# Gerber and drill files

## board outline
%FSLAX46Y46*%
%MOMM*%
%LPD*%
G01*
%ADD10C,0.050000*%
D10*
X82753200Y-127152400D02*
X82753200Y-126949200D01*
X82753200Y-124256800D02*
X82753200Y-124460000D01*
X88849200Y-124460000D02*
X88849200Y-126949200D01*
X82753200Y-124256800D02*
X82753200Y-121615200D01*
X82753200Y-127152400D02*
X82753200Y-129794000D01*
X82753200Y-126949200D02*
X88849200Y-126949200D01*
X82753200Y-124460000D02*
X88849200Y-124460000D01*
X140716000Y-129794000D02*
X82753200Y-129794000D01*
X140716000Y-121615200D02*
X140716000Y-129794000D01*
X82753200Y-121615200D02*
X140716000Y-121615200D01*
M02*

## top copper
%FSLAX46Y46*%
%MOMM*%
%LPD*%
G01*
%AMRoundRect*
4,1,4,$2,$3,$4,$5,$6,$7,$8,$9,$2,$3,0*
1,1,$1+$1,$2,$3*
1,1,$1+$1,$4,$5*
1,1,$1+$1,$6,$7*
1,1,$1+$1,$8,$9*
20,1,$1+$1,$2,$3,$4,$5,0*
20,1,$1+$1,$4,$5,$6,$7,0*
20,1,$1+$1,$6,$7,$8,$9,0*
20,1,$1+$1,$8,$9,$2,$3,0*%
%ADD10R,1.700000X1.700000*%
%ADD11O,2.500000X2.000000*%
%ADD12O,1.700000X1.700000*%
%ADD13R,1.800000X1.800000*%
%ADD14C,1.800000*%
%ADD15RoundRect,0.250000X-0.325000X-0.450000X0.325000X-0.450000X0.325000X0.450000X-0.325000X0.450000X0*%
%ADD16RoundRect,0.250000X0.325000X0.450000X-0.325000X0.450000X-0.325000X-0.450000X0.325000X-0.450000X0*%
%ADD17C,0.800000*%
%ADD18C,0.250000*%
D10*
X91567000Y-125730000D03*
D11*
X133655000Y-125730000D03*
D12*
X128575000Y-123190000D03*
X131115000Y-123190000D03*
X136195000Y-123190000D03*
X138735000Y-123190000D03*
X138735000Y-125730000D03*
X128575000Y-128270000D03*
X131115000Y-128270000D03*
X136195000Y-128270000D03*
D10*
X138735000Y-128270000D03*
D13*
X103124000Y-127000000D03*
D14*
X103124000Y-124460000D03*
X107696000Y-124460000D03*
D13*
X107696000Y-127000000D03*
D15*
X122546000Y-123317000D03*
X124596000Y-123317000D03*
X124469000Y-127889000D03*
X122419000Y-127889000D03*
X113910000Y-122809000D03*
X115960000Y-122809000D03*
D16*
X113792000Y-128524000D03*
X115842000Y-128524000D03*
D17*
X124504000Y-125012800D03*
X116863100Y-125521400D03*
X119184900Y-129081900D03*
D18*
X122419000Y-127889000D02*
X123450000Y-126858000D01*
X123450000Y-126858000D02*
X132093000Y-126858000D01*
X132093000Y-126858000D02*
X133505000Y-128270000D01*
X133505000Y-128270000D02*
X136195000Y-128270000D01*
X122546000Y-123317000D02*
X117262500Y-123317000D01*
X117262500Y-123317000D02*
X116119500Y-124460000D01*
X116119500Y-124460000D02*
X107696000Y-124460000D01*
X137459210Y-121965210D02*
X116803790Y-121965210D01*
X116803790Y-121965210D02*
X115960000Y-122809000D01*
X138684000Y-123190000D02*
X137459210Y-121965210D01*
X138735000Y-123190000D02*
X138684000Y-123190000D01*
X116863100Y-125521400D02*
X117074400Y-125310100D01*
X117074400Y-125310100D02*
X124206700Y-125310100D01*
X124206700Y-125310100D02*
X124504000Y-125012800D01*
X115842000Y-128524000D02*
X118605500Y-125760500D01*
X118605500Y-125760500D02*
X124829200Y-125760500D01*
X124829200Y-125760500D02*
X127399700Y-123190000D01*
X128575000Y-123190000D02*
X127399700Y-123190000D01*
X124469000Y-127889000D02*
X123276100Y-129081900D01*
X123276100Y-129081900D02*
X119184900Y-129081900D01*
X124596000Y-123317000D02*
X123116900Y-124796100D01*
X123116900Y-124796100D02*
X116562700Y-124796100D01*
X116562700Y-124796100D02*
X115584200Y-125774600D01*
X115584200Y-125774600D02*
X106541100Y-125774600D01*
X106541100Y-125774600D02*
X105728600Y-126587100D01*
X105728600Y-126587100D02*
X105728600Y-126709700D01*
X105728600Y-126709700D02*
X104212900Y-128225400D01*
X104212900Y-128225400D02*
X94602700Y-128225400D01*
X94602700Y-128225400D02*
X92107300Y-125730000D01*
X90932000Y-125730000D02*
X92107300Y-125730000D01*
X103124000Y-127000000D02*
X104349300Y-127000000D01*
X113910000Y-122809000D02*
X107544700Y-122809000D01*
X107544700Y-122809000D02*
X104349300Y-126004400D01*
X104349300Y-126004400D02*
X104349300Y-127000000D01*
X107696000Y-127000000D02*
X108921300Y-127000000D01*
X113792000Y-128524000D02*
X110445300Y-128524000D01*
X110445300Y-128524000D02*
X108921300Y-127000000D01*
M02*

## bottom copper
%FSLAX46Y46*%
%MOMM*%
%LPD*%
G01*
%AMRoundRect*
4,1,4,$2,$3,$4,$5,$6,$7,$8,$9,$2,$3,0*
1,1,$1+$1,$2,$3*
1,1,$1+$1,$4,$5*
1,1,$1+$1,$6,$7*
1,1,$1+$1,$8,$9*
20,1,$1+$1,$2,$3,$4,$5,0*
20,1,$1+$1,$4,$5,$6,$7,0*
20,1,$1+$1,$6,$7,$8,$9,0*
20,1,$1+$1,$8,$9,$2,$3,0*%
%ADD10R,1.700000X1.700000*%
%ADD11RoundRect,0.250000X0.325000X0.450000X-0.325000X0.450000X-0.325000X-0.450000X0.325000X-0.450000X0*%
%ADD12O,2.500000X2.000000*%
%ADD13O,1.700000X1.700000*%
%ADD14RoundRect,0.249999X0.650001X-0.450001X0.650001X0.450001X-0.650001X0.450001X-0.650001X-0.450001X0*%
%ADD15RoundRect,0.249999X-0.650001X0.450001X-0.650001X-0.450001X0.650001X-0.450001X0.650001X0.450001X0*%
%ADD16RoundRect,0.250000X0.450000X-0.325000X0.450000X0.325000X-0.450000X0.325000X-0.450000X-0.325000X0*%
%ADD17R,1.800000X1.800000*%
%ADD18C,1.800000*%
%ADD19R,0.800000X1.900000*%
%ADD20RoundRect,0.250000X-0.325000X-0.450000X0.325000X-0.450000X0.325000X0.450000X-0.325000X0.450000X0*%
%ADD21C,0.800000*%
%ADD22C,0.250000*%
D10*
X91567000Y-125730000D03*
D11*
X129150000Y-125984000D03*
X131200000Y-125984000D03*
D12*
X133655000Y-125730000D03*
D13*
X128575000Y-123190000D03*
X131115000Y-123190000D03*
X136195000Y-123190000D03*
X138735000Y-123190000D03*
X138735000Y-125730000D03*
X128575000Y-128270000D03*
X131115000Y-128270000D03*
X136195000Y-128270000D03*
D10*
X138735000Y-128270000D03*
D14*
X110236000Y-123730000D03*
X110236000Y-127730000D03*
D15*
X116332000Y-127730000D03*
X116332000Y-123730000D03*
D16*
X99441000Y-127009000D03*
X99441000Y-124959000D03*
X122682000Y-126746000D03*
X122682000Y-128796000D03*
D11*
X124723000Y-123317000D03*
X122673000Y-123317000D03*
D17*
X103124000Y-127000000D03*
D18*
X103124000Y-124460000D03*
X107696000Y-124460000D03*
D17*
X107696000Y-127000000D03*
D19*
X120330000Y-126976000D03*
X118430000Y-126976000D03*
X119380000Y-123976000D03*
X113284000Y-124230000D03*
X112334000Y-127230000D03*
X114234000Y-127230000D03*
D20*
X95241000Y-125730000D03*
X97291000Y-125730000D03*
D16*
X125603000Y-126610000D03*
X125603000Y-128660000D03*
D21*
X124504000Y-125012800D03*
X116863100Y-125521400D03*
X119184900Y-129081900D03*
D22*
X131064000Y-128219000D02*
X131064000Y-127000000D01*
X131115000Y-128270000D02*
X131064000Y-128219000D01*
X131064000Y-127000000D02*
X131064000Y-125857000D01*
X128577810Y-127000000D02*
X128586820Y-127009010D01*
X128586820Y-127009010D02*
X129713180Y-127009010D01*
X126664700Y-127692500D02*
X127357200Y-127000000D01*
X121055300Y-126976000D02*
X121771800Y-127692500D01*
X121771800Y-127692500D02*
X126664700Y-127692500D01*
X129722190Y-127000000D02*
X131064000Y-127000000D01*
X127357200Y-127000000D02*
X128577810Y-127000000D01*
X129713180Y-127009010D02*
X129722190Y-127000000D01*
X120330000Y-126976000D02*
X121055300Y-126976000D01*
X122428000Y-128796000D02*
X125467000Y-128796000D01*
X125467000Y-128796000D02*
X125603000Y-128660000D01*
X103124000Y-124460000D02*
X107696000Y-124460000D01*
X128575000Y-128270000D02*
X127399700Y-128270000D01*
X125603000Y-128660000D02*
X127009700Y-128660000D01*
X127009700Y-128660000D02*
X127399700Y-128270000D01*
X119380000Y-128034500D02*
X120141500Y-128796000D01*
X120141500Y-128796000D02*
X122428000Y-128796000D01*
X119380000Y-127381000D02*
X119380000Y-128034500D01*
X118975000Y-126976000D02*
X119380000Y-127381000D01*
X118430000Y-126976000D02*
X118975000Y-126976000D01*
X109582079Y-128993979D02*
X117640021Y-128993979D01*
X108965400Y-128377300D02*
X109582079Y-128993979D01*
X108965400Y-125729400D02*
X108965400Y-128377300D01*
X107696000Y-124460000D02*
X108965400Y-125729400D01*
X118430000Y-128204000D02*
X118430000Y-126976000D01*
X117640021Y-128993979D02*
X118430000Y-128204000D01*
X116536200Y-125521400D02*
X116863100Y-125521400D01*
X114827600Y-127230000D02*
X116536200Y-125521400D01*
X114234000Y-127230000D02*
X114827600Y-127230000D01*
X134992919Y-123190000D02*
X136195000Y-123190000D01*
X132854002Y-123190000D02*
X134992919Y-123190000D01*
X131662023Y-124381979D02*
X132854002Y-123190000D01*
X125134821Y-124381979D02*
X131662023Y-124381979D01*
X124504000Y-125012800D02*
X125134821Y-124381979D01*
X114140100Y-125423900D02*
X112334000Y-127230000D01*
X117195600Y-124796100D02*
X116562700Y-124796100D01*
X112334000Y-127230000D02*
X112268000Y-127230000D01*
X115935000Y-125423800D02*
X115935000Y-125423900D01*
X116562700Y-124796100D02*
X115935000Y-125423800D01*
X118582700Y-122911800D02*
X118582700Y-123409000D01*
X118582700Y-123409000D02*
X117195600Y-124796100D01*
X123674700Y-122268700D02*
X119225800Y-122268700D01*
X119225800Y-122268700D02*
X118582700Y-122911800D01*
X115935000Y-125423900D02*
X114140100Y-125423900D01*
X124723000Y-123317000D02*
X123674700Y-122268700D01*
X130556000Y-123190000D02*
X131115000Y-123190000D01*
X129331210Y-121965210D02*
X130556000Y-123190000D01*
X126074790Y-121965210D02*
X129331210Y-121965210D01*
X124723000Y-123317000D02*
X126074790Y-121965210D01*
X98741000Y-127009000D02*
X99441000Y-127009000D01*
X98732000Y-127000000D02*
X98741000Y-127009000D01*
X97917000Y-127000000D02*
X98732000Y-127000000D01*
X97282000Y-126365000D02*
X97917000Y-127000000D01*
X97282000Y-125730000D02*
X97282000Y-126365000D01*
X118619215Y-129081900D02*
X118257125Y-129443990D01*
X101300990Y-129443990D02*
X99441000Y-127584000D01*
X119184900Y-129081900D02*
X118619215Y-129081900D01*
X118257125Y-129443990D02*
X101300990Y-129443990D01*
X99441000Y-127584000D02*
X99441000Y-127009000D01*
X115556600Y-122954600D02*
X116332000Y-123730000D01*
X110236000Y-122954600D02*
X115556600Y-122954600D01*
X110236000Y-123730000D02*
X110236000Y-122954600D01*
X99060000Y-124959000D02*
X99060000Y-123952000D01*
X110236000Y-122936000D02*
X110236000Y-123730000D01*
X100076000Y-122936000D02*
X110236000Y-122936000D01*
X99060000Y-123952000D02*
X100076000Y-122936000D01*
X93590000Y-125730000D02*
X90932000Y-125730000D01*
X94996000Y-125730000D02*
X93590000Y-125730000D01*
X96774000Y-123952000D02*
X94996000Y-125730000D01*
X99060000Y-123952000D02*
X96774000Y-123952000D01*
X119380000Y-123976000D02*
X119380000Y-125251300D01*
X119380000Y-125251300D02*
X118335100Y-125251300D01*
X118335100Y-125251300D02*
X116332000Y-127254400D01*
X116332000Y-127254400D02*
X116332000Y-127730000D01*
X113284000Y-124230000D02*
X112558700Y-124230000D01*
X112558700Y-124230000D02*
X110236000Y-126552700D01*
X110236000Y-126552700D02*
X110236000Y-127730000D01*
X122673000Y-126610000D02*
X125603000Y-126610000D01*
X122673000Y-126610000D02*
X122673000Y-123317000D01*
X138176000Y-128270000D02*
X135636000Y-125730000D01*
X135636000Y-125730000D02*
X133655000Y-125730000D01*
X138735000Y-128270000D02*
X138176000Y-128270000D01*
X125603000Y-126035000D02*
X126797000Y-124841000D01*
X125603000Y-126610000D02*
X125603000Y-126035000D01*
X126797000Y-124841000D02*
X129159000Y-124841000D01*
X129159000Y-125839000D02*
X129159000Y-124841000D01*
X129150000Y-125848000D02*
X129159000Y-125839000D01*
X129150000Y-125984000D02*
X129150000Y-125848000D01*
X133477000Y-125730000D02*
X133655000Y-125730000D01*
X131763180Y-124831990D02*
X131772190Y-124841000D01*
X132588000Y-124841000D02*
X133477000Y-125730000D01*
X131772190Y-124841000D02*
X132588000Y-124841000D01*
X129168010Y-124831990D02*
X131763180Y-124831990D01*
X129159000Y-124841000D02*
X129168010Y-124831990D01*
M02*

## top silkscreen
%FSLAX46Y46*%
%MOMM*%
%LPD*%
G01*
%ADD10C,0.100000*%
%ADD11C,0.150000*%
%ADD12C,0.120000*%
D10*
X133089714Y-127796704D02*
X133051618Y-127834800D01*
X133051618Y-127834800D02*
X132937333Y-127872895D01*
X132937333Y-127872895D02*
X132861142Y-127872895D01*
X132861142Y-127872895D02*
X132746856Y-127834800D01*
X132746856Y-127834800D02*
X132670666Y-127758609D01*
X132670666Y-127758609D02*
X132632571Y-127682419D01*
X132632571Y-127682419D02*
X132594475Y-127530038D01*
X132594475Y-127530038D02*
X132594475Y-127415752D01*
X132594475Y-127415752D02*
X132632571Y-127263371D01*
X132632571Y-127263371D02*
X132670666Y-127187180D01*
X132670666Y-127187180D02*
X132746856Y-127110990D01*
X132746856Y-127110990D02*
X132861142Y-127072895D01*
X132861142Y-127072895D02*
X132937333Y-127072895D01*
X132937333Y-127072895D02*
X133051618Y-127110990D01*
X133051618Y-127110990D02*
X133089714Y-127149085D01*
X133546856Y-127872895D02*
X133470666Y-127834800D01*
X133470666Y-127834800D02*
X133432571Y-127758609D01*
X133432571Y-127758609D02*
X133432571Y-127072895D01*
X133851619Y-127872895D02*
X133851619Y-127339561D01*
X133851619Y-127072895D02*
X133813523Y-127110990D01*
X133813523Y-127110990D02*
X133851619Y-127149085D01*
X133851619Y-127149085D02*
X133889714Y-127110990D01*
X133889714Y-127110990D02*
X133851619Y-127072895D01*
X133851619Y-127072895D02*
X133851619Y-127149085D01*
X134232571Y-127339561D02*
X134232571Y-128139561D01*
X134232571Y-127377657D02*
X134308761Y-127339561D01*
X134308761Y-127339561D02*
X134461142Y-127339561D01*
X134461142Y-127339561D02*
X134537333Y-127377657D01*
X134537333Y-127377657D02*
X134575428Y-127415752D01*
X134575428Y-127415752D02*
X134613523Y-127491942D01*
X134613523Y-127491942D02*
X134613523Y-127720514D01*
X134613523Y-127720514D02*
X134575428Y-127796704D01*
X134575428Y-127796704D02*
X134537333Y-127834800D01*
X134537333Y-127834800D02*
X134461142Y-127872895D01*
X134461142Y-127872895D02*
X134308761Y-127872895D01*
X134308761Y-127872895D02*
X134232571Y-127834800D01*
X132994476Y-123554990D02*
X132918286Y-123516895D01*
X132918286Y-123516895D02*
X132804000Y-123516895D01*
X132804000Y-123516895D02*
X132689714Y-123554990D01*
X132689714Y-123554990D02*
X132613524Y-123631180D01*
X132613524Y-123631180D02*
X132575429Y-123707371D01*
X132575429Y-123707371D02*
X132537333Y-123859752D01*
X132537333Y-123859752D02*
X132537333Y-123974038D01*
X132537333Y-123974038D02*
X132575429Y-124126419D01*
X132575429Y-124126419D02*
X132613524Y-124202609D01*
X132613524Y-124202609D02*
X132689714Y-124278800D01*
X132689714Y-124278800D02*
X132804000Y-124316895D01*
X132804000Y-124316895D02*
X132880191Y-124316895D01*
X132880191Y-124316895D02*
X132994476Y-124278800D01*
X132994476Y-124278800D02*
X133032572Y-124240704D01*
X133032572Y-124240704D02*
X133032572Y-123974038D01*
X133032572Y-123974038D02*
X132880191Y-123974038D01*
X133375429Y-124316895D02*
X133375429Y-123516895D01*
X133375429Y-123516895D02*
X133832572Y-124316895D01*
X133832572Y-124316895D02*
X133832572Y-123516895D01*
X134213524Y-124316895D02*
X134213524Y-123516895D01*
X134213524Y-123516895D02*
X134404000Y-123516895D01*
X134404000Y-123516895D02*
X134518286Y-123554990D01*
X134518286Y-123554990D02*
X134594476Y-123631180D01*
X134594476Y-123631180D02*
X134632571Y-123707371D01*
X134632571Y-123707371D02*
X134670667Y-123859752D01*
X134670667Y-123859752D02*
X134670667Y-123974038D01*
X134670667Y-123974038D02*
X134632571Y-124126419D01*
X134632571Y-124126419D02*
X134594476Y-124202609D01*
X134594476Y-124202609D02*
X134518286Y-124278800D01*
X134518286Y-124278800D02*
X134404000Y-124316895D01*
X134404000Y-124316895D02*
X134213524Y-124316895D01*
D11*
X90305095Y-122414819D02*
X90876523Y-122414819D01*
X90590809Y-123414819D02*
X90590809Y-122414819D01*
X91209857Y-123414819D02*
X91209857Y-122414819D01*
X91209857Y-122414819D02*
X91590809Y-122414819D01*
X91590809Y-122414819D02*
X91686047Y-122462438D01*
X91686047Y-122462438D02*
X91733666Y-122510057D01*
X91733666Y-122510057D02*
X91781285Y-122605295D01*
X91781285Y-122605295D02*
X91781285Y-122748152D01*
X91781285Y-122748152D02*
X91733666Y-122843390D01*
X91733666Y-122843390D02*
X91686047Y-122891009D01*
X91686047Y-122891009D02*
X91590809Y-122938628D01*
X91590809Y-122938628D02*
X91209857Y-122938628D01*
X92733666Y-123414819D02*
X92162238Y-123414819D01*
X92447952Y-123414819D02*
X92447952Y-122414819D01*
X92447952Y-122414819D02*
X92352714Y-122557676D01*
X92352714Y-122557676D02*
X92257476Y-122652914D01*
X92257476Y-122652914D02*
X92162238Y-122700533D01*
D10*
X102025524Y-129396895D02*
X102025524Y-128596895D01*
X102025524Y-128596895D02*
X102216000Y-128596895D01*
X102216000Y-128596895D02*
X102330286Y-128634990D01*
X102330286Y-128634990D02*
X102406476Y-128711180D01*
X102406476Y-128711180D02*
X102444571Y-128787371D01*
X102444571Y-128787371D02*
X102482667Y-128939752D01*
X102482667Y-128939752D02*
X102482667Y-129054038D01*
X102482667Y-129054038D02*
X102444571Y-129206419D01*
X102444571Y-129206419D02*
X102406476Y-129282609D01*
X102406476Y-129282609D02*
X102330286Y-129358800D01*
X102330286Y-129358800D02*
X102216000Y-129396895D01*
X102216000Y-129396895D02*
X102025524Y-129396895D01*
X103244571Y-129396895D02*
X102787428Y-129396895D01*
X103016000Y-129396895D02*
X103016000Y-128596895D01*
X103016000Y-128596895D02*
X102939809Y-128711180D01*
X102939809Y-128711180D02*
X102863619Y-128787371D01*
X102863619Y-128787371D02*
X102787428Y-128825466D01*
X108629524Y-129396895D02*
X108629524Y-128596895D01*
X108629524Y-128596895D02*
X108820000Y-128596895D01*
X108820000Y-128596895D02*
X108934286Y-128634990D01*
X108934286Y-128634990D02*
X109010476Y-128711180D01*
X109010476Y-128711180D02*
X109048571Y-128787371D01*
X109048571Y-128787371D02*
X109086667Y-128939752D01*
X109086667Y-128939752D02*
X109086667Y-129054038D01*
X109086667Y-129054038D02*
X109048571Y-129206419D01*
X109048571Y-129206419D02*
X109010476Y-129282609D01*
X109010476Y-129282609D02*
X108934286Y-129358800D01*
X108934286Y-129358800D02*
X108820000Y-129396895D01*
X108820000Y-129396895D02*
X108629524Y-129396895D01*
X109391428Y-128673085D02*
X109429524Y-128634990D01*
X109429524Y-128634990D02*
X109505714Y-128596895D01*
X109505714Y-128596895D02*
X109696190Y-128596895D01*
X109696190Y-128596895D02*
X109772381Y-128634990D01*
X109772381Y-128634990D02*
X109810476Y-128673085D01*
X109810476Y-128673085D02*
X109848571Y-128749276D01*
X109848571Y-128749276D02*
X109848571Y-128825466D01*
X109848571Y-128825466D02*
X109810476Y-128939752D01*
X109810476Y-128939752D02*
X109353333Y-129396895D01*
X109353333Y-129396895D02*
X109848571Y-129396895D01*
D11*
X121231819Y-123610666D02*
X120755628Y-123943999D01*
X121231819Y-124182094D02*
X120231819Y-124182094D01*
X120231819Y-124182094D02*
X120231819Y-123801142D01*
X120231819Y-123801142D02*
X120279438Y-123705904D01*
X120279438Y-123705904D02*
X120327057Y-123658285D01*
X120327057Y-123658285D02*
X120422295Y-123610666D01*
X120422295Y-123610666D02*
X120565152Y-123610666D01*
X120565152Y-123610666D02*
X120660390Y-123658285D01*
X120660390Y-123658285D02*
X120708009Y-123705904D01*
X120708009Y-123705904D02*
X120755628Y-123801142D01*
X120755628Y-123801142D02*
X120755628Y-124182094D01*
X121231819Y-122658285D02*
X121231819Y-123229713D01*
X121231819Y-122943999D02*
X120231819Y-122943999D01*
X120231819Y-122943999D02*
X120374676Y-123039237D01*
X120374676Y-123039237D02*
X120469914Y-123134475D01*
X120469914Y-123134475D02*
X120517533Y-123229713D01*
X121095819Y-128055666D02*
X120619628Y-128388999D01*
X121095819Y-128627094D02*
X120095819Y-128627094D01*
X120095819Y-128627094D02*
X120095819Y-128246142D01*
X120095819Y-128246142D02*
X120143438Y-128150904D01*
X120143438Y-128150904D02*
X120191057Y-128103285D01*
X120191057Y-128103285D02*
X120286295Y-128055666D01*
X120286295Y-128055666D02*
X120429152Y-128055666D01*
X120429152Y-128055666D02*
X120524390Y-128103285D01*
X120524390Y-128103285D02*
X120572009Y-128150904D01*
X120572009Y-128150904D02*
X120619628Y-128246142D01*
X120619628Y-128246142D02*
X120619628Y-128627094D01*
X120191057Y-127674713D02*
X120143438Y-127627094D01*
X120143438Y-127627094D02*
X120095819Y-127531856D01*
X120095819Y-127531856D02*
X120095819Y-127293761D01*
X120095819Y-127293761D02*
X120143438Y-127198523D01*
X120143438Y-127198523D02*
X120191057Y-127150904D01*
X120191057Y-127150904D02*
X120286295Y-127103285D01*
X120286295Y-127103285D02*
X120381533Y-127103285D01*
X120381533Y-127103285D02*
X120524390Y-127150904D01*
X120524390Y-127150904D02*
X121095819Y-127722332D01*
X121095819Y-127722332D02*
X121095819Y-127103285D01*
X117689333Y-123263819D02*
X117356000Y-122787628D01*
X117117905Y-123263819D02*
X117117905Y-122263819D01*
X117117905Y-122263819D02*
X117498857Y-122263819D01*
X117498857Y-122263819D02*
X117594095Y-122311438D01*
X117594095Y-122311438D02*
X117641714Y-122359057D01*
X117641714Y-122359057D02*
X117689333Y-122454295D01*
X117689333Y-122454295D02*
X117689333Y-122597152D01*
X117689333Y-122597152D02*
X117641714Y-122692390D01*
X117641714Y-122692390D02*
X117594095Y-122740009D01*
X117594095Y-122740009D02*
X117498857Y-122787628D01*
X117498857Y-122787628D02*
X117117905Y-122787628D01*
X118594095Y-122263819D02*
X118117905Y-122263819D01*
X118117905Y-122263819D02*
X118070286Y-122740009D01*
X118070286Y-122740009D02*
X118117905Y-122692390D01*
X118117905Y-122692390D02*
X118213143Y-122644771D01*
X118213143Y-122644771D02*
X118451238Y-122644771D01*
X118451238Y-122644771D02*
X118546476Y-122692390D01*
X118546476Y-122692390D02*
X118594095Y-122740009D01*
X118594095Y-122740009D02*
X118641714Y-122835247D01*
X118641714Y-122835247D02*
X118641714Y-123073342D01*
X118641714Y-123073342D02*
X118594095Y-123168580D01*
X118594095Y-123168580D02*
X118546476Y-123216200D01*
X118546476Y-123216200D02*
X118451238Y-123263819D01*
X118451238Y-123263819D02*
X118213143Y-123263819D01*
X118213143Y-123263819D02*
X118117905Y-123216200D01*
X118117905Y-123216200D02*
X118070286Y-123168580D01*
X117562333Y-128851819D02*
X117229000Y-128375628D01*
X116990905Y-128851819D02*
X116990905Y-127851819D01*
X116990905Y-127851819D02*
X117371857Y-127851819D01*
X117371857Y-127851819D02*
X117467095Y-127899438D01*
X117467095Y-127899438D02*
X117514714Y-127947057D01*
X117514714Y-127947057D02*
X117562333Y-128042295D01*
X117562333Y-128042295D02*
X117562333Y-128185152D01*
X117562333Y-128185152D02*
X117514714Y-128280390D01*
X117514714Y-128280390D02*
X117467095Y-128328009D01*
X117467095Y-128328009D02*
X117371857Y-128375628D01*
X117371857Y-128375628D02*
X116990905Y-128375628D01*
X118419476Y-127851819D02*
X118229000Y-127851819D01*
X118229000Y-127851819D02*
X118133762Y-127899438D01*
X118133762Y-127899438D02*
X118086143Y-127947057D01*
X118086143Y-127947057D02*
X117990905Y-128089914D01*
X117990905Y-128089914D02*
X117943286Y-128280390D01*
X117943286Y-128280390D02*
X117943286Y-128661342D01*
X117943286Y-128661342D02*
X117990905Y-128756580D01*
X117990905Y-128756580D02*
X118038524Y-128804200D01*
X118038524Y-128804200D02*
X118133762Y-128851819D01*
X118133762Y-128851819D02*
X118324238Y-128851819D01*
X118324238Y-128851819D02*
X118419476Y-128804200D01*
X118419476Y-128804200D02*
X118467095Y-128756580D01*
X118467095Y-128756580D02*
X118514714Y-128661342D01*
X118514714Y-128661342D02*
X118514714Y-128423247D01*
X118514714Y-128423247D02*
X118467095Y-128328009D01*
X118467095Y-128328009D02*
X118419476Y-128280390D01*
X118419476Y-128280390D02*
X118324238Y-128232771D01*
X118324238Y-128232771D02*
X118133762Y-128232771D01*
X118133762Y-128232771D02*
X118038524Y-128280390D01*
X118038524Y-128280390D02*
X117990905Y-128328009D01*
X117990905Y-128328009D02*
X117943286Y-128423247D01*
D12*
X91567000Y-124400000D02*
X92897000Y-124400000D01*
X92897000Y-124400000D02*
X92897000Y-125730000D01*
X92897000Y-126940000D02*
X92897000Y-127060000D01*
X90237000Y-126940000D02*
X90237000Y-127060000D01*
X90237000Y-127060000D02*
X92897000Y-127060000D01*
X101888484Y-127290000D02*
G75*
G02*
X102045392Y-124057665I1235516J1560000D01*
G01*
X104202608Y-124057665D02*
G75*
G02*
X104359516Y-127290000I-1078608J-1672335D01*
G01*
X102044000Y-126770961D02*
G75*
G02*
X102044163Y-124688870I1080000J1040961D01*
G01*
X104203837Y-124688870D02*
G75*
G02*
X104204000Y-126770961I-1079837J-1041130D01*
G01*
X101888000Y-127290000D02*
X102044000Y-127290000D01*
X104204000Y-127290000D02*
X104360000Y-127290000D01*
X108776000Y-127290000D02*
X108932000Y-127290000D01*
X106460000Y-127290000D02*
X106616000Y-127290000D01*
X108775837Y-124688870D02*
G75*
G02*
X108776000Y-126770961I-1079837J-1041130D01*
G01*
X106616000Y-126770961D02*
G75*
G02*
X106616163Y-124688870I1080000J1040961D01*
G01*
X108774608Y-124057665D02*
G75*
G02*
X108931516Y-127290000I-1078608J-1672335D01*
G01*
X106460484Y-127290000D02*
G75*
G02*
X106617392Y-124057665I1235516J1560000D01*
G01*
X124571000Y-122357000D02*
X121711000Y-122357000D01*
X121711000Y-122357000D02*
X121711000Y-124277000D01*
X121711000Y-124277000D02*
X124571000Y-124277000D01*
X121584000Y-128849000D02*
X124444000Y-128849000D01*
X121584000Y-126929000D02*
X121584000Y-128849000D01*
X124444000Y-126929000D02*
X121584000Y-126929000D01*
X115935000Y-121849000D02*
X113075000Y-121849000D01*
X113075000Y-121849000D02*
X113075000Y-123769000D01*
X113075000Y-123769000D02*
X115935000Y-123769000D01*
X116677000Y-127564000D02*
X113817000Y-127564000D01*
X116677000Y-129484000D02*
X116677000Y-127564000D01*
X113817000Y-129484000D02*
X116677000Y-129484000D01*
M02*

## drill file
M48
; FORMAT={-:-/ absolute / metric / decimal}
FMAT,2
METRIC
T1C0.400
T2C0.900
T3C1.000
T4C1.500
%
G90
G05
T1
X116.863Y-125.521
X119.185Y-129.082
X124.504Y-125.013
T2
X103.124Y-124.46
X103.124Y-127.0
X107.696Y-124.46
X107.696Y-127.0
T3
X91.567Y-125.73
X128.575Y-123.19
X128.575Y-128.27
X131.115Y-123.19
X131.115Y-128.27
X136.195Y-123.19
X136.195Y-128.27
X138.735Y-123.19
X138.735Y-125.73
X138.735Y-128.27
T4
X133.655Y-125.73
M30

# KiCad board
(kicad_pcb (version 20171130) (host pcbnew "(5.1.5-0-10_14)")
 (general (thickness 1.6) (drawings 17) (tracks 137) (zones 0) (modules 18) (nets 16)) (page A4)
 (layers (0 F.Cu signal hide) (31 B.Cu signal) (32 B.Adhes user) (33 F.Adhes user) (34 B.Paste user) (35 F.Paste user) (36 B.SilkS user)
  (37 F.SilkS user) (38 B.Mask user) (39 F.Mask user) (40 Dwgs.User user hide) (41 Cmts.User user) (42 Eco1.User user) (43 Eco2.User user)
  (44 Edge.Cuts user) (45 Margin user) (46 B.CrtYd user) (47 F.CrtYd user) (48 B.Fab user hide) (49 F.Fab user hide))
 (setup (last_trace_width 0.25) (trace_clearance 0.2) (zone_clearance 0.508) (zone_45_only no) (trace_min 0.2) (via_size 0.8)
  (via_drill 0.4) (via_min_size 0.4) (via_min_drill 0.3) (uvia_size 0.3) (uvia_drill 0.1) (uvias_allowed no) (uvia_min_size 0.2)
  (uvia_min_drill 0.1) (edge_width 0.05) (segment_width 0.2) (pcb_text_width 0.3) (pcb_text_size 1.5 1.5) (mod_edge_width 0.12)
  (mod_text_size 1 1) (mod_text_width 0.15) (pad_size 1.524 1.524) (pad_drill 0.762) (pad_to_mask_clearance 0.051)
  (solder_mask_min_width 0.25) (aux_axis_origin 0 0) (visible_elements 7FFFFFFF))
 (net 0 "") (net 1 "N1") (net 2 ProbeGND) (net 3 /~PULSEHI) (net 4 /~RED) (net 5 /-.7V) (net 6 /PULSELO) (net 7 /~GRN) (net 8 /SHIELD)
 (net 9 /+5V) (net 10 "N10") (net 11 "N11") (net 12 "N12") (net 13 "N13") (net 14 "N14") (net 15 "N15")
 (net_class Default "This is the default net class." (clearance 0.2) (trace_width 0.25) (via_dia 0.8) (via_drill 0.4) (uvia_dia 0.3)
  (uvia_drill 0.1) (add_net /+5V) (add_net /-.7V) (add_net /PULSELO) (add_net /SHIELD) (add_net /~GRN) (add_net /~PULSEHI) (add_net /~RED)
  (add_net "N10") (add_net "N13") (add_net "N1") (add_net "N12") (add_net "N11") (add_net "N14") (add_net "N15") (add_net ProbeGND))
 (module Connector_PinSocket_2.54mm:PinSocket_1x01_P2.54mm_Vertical (layer F.Cu) (at 91.567 125.73)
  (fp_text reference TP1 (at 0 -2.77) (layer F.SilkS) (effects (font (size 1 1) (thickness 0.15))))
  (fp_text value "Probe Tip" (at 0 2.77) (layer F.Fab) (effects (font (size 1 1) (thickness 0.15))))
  (fp_line (start 0 -1.33) (end 1.33 -1.33) (layer F.SilkS) (width 0.12))
  (fp_line (start 1.33 -1.33) (end 1.33 0) (layer F.SilkS) (width 0.12))
  (fp_line (start 1.33 1.21) (end 1.33 1.33) (layer F.SilkS) (width 0.12))
  (fp_line (start -1.33 1.21) (end -1.33 1.33) (layer F.SilkS) (width 0.12))
  (fp_line (start -1.33 1.33) (end 1.33 1.33) (layer F.SilkS) (width 0.12))
  (pad 1 thru_hole rect (at 0 0) (size 1.7 1.7) (drill 1) (layers *.Cu *.Mask) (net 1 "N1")))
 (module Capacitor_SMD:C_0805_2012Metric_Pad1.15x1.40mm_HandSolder (layer B.Cu) (at 130.175 125.984 180)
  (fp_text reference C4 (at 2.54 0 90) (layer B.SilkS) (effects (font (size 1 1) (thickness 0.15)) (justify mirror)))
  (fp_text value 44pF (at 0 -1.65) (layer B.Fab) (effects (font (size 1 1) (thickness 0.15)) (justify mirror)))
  (pad 2 smd roundrect (at 1.025 0 180) (size 1.15 1.4) (layers B.Cu B.Paste B.Mask) (roundrect_rratio 0.217391) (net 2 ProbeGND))
  (pad 1 smd roundrect (at -1.025 0 180) (size 1.15 1.4) (layers B.Cu B.Paste B.Mask) (roundrect_rratio 0.217391) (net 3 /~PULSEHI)))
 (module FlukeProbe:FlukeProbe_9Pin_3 (layer B.Cu) (at 138.735 128.27 90)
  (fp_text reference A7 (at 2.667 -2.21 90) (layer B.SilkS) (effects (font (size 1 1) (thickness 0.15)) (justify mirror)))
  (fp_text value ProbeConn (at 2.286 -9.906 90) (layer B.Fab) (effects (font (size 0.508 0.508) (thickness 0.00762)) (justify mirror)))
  (pad 10 thru_hole oval (at 2.54 -5.08 90) (size 2 2.5) (drill 1.5) (layers *.Cu *.Mask) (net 2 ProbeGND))
  (pad 9 thru_hole oval (at 5.08 -10.16 90) (size 1.7 1.7) (drill 1) (layers *.Cu *.Mask) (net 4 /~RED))
  (pad 8 thru_hole oval (at 5.08 -7.62 90) (size 1.7 1.7) (drill 1) (layers *.Cu *.Mask) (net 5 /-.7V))
  (pad 7 thru_hole oval (at 5.08 -2.54 90) (size 1.7 1.7) (drill 1) (layers *.Cu *.Mask) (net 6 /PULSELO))
  (pad 6 thru_hole oval (at 5.08 0 90) (size 1.7 1.7) (drill 1) (layers *.Cu *.Mask) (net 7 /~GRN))
  (pad 5 thru_hole oval (at 2.54 0 90) (size 1.7 1.7) (drill 1) (layers *.Cu *.Mask) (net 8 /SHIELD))
  (pad 4 thru_hole oval (at 0 -10.16 90) (size 1.7 1.7) (drill 1) (layers *.Cu *.Mask) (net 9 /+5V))
  (pad 3 thru_hole oval (at 0 -7.62 90) (size 1.7 1.7) (drill 1) (layers *.Cu *.Mask) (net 3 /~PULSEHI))
  (pad 2 thru_hole oval (at 0 -2.54 90) (size 1.7 1.7) (drill 1) (layers *.Cu *.Mask) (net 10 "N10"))
  (pad 1 thru_hole rect (at 0 0 90) (size 1.7 1.7) (drill 1) (layers *.Cu *.Mask) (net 2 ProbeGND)))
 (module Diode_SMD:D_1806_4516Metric (layer B.Cu) (at 110.236 125.73 90)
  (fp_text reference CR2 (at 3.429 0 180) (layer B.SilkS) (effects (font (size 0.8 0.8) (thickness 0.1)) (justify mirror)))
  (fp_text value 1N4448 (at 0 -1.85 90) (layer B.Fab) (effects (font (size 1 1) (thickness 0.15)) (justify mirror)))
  (pad 2 smd roundrect (at 2 0 90) (size 1.4 1.8) (layers B.Cu B.Paste B.Mask) (roundrect_rratio 0.178571) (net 1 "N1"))
  (pad 1 smd roundrect (at -2 0 90) (size 1.4 1.8) (layers B.Cu B.Paste B.Mask) (roundrect_rratio 0.178571) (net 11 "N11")))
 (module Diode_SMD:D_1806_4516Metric (layer B.Cu) (at 116.332 125.73 270)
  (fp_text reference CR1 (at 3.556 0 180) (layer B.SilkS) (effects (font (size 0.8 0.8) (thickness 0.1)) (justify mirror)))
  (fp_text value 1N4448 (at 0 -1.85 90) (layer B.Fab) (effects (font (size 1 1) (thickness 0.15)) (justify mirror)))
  (pad 2 smd roundrect (at 2 0 270) (size 1.4 1.8) (layers B.Cu B.Paste B.Mask) (roundrect_rratio 0.178571) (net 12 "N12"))
  (pad 1 smd roundrect (at -2 0 270) (size 1.4 1.8) (layers B.Cu B.Paste B.Mask) (roundrect_rratio 0.178571) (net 1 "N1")))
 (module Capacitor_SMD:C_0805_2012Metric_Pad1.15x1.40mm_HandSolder (layer B.Cu) (at 99.441 125.984 90)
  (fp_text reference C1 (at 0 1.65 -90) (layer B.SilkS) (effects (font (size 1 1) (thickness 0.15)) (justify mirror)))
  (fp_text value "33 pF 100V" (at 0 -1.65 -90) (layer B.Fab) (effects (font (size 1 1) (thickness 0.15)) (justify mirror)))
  (pad 1 smd roundrect (at -1.025 0 90) (size 1.15 1.4) (layers B.Cu B.Paste B.Mask) (roundrect_rratio 0.217391) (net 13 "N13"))
  (pad 2 smd roundrect (at 1.025 0 90) (size 1.15 1.4) (layers B.Cu B.Paste B.Mask) (roundrect_rratio 0.217391) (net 1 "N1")))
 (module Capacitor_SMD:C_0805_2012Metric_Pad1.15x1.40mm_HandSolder (layer B.Cu) (at 122.682 127.771 90)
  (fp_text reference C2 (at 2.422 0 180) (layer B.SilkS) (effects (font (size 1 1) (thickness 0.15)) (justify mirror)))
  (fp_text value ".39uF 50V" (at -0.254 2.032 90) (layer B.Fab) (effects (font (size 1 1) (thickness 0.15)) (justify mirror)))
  (pad 2 smd roundrect (at 1.025 0 90) (size 1.15 1.4) (layers B.Cu B.Paste B.Mask) (roundrect_rratio 0.217391) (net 2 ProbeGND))
  (pad 1 smd roundrect (at -1.025 0 90) (size 1.15 1.4) (layers B.Cu B.Paste B.Mask) (roundrect_rratio 0.217391) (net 9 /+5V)))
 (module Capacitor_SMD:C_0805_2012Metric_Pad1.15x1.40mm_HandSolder (layer B.Cu) (at 123.698 123.317 180)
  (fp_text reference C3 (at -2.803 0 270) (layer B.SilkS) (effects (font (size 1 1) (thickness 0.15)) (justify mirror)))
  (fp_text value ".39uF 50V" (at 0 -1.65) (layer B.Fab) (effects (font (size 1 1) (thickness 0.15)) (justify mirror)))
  (pad 1 smd roundrect (at -1.025 0 180) (size 1.15 1.4) (layers B.Cu B.Paste B.Mask) (roundrect_rratio 0.217391) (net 5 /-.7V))
  (pad 2 smd roundrect (at 1.025 0 180) (size 1.15 1.4) (layers B.Cu B.Paste B.Mask) (roundrect_rratio 0.217391) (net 2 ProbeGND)))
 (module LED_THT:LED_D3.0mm (layer F.Cu) (at 103.124 127 90)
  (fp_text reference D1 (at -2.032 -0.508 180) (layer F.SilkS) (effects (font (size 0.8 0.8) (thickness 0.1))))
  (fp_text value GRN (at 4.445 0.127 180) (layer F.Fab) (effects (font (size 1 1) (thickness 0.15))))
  (fp_arc (start 1.27 0) (end -0.29 -1.235516) (angle 108.8) (layer F.SilkS) (width 0.12))
  (fp_arc (start 1.27 0) (end -0.29 1.235516) (angle -108.8) (layer F.SilkS) (width 0.12))
  (fp_arc (start 1.27 0) (end 0.229039 -1.08) (angle 87.9) (layer F.SilkS) (width 0.12))
  (fp_arc (start 1.27 0) (end 0.229039 1.08) (angle -87.9) (layer F.SilkS) (width 0.12))
  (fp_line (start -0.29 -1.236) (end -0.29 -1.08) (layer F.SilkS) (width 0.12))
  (fp_line (start -0.29 1.08) (end -0.29 1.236) (layer F.SilkS) (width 0.12))
  (pad 1 thru_hole rect (at 0 0 90) (size 1.8 1.8) (drill 0.9) (layers *.Cu *.Mask) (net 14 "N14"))
  (pad 2 thru_hole circle (at 2.54 0 90) (size 1.8 1.8) (drill 0.9) (layers *.Cu *.Mask) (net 9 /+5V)))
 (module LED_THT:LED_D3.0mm (layer F.Cu) (at 107.696 127 90)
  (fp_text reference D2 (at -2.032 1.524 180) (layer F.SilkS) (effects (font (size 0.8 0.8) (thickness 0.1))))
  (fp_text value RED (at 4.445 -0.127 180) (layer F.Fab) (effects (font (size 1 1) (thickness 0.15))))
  (fp_line (start -0.29 1.08) (end -0.29 1.236) (layer F.SilkS) (width 0.12))
  (fp_line (start -0.29 -1.236) (end -0.29 -1.08) (layer F.SilkS) (width 0.12))
  (fp_arc (start 1.27 0) (end 0.229039 1.08) (angle -87.9) (layer F.SilkS) (width 0.12))
  (fp_arc (start 1.27 0) (end 0.229039 -1.08) (angle 87.9) (layer F.SilkS) (width 0.12))
  (fp_arc (start 1.27 0) (end -0.29 1.235516) (angle -108.8) (layer F.SilkS) (width 0.12))
  (fp_arc (start 1.27 0) (end -0.29 -1.235516) (angle 108.8) (layer F.SilkS) (width 0.12))
  (pad 2 thru_hole circle (at 2.54 0 90) (size 1.8 1.8) (drill 0.9) (layers *.Cu *.Mask) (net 9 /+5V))
  (pad 1 thru_hole rect (at 0 0 90) (size 1.8 1.8) (drill 0.9) (layers *.Cu *.Mask) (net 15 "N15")))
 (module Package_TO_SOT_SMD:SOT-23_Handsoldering (layer B.Cu) (at 119.38 125.476 90)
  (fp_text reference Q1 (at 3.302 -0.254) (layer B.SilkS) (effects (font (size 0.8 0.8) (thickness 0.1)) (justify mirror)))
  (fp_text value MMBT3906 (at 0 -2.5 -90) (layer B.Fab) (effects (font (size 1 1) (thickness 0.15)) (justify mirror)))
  (pad 1 smd rect (at -1.5 0.95 90) (size 1.9 0.8) (layers B.Cu B.Paste B.Mask) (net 3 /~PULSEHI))
  (pad 2 smd rect (at -1.5 -0.95 90) (size 1.9 0.8) (layers B.Cu B.Paste B.Mask) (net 9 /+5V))
  (pad 3 smd rect (at 1.5 0 90) (size 1.9 0.8) (layers B.Cu B.Paste B.Mask) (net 12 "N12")))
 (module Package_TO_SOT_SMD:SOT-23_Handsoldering (layer B.Cu) (at 113.284 125.73 90)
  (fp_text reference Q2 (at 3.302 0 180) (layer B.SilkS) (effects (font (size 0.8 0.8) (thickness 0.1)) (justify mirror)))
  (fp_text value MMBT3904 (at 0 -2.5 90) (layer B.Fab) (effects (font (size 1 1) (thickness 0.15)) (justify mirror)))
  (pad 3 smd rect (at 1.5 0 90) (size 1.9 0.8) (layers B.Cu B.Paste B.Mask) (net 11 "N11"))
  (pad 2 smd rect (at -1.5 -0.95 90) (size 1.9 0.8) (layers B.Cu B.Paste B.Mask) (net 5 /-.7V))
  (pad 1 smd rect (at -1.5 0.95 90) (size 1.9 0.8) (layers B.Cu B.Paste B.Mask) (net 6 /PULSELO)))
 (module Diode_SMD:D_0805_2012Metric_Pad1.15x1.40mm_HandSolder (layer F.Cu) (at 123.571 123.317)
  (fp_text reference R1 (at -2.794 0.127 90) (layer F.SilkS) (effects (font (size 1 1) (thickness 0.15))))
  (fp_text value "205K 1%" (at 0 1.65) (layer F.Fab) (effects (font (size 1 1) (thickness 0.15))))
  (fp_line (start 1 -0.96) (end -1.86 -0.96) (layer F.SilkS) (width 0.12))
  (fp_line (start -1.86 -0.96) (end -1.86 0.96) (layer F.SilkS) (width 0.12))
  (fp_line (start -1.86 0.96) (end 1 0.96) (layer F.SilkS) (width 0.12))
  (pad 1 smd roundrect (at -1.025 0) (size 1.15 1.4) (layers F.Cu F.Paste F.Mask) (roundrect_rratio 0.217391) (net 9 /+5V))
  (pad 2 smd roundrect (at 1.025 0) (size 1.15 1.4) (layers F.Cu F.Paste F.Mask) (roundrect_rratio 0.217391) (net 1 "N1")))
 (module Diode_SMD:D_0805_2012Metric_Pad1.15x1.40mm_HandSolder (layer F.Cu) (at 123.444 127.889)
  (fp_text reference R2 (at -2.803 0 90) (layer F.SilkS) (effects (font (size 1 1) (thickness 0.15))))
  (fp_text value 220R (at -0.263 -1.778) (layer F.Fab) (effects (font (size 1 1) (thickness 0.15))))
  (fp_line (start -1.86 0.96) (end 1 0.96) (layer F.SilkS) (width 0.12))
  (fp_line (start -1.86 -0.96) (end -1.86 0.96) (layer F.SilkS) (width 0.12))
  (fp_line (start 1 -0.96) (end -1.86 -0.96) (layer F.SilkS) (width 0.12))
  (pad 2 smd roundrect (at 1.025 0) (size 1.15 1.4) (layers F.Cu F.Paste F.Mask) (roundrect_rratio 0.217391) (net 13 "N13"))
  (pad 1 smd roundrect (at -1.025 0) (size 1.15 1.4) (layers F.Cu F.Paste F.Mask) (roundrect_rratio 0.217391) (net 10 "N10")))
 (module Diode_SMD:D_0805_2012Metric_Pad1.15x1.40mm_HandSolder (layer B.Cu) (at 96.266 125.73)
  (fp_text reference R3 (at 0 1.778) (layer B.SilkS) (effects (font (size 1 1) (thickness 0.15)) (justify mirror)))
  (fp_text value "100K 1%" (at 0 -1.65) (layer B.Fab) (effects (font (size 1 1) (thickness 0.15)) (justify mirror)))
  (pad 1 smd roundrect (at -1.025 0) (size 1.15 1.4) (layers B.Cu B.Paste B.Mask) (roundrect_rratio 0.217391) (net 1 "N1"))
  (pad 2 smd roundrect (at 1.025 0) (size 1.15 1.4) (layers B.Cu B.Paste B.Mask) (roundrect_rratio 0.217391) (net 13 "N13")))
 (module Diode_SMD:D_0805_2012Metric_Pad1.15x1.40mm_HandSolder (layer B.Cu) (at 125.603 127.635 90)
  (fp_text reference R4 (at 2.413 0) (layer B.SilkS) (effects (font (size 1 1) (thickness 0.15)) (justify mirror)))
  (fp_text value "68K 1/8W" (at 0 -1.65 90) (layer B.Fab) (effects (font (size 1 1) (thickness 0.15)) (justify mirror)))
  (pad 2 smd roundrect (at 1.025 0 90) (size 1.15 1.4) (layers B.Cu B.Paste B.Mask) (roundrect_rratio 0.217391) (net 2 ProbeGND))
  (pad 1 smd roundrect (at -1.025 0 90) (size 1.15 1.4) (layers B.Cu B.Paste B.Mask) (roundrect_rratio 0.217391) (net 9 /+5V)))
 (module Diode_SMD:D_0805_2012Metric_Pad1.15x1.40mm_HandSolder (layer F.Cu) (at 114.935 122.809)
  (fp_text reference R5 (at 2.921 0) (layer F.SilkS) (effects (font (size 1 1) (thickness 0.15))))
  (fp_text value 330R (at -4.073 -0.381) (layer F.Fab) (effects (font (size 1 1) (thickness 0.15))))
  (fp_line (start 1 -0.96) (end -1.86 -0.96) (layer F.SilkS) (width 0.12))
  (fp_line (start -1.86 -0.96) (end -1.86 0.96) (layer F.SilkS) (width 0.12))
  (fp_line (start -1.86 0.96) (end 1 0.96) (layer F.SilkS) (width 0.12))
  (pad 1 smd roundrect (at -1.025 0) (size 1.15 1.4) (layers F.Cu F.Paste F.Mask) (roundrect_rratio 0.217391) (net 14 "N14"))
  (pad 2 smd roundrect (at 1.025 0) (size 1.15 1.4) (layers F.Cu F.Paste F.Mask) (roundrect_rratio 0.217391) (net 7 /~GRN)))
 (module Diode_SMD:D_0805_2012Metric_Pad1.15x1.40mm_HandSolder (layer F.Cu) (at 114.817 128.524 180)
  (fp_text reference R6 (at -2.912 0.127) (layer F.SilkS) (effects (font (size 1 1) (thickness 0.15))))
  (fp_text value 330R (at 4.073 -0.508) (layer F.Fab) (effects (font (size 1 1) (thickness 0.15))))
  (fp_line (start -1.86 0.96) (end 1 0.96) (layer F.SilkS) (width 0.12))
  (fp_line (start -1.86 -0.96) (end -1.86 0.96) (layer F.SilkS) (width 0.12))
  (fp_line (start 1 -0.96) (end -1.86 -0.96) (layer F.SilkS) (width 0.12))
  (pad 2 smd roundrect (at 1.025 0 180) (size 1.15 1.4) (layers F.Cu F.Paste F.Mask) (roundrect_rratio 0.217391) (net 15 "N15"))
  (pad 1 smd roundrect (at -1.025 0 180) (size 1.15 1.4) (layers F.Cu F.Paste F.Mask) (roundrect_rratio 0.217391) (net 4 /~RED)))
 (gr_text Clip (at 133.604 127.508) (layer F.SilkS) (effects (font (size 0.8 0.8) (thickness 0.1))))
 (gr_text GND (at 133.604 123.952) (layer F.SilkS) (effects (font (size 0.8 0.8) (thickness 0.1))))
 (gr_line (start 82.7532 127.1524) (end 82.7532 126.9492) (layer Edge.Cuts) (width 0.05))
 (gr_line (start 82.7532 124.2568) (end 82.7532 124.46) (layer Edge.Cuts) (width 0.05))
 (gr_line (start 88.8492 124.46) (end 88.8492 126.9492) (layer Edge.Cuts) (width 0.05))
 (gr_line (start 82.7532 124.2568) (end 82.7532 121.6152) (layer Edge.Cuts) (width 0.05))
 (gr_line (start 82.7532 127.1524) (end 82.7532 129.794) (layer Edge.Cuts) (width 0.05))
 (gr_line (start 82.7532 126.9492) (end 88.8492 126.9492) (layer Edge.Cuts) (width 0.05))
 (gr_line (start 82.7532 124.46) (end 88.8492 124.46) (layer Edge.Cuts) (width 0.05))
 (gr_line (start 140.716 129.794) (end 82.7532 129.794) (layer Edge.Cuts) (width 0.05))
 (gr_line (start 140.716 121.6152) (end 140.716 129.794) (layer Edge.Cuts) (width 0.05))
 (gr_line (start 82.7532 121.6152) (end 140.716 121.6152) (layer Edge.Cuts) (width 0.05))
 (segment (start 122.419 127.889) (end 123.45 126.858) (width 0.25) (layer F.Cu) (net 10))
 (segment (start 123.45 126.858) (end 132.093 126.858) (width 0.25) (layer F.Cu) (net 10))
 (segment (start 132.093 126.858) (end 133.505 128.27) (width 0.25) (layer F.Cu) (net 10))
 (segment (start 133.505 128.27) (end 136.195 128.27) (width 0.25) (layer F.Cu) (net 10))
 (segment (start 131.064 128.219) (end 131.064 127) (width 0.25) (layer B.Cu) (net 3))
 (segment (start 131.115 128.27) (end 131.064 128.219) (width 0.25) (layer B.Cu) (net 3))
 (segment (start 131.064 127) (end 131.064 125.857) (width 0.25) (layer B.Cu) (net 3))
 (segment (start 128.57781 127) (end 128.58682 127.00901) (width 0.25) (layer B.Cu) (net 3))
 (segment (start 128.58682 127.00901) (end 129.71318 127.00901) (width 0.25) (layer B.Cu) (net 3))
 (segment (start 126.6647 127.6925) (end 127.3572 127) (width 0.25) (layer B.Cu) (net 3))
 (segment (start 121.0553 126.976) (end 121.7718 127.6925) (width 0.25) (layer B.Cu) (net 3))
 (segment (start 121.7718 127.6925) (end 126.6647 127.6925) (width 0.25) (layer B.Cu) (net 3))
 (segment (start 129.72219 127) (end 131.064 127) (width 0.25) (layer B.Cu) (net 3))
 (segment (start 127.3572 127) (end 128.57781 127) (width 0.25) (layer B.Cu) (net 3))
 (segment (start 129.71318 127.00901) (end 129.72219 127) (width 0.25) (layer B.Cu) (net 3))
 (segment (start 120.33 126.976) (end 121.0553 126.976) (width 0.25) (layer B.Cu) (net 3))
 (segment (start 122.546 123.317) (end 117.2625 123.317) (width 0.25) (layer F.Cu) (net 9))
 (segment (start 117.2625 123.317) (end 116.1195 124.46) (width 0.25) (layer F.Cu) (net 9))
 (segment (start 116.1195 124.46) (end 107.696 124.46) (width 0.25) (layer F.Cu) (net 9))
 (segment (start 122.428 128.796) (end 125.467 128.796) (width 0.25) (layer B.Cu) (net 9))
 (segment (start 125.467 128.796) (end 125.603 128.66) (width 0.25) (layer B.Cu) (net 9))
 (segment (start 103.124 124.46) (end 107.696 124.46) (width 0.25) (layer B.Cu) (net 9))
 (segment (start 128.575 128.27) (end 127.3997 128.27) (width 0.25) (layer B.Cu) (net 9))
 (segment (start 125.603 128.66) (end 127.0097 128.66) (width 0.25) (layer B.Cu) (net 9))
 (segment (start 127.0097 128.66) (end 127.3997 128.27) (width 0.25) (layer B.Cu) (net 9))
 (segment (start 119.38 128.0345) (end 120.1415 128.796) (width 0.25) (layer B.Cu) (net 9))
 (segment (start 120.1415 128.796) (end 122.428 128.796) (width 0.25) (layer B.Cu) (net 9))
 (segment (start 119.38 127.381) (end 119.38 128.0345) (width 0.25) (layer B.Cu) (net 9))
 (segment (start 118.975 126.976) (end 119.38 127.381) (width 0.25) (layer B.Cu) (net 9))
 (segment (start 118.43 126.976) (end 118.975 126.976) (width 0.25) (layer B.Cu) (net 9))
 (segment (start 109.582079 128.993979) (end 117.640021 128.993979) (width 0.25) (layer B.Cu) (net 9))
 (segment (start 108.9654 128.3773) (end 109.582079 128.993979) (width 0.25) (layer B.Cu) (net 9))
 (segment (start 108.9654 125.7294) (end 108.9654 128.3773) (width 0.25) (layer B.Cu) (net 9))
 (segment (start 107.696 124.46) (end 108.9654 125.7294) (width 0.25) (layer B.Cu) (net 9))
 (segment (start 118.43 128.204) (end 118.43 126.976) (width 0.25) (layer B.Cu) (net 9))
 (segment (start 117.640021 128.993979) (end 118.43 128.204) (width 0.25) (layer B.Cu) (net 9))
 (segment (start 137.45921 121.96521) (end 116.80379 121.96521) (width 0.25) (layer F.Cu) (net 7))
 (segment (start 116.80379 121.96521) (end 115.96 122.809) (width 0.25) (layer F.Cu) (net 7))
 (segment (start 138.684 123.19) (end 137.45921 121.96521) (width 0.25) (layer F.Cu) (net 7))
 (segment (start 138.735 123.19) (end 138.684 123.19) (width 0.25) (layer F.Cu) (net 7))
 (segment (start 116.8631 125.5214) (end 117.0744 125.3101) (width 0.25) (layer F.Cu) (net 6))
 (segment (start 117.0744 125.3101) (end 124.2067 125.3101) (width 0.25) (layer F.Cu) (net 6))
 (segment (start 124.2067 125.3101) (end 124.504 125.0128) (width 0.25) (layer F.Cu) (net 6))
 (via (at 124.504 125.0128) (size 0.8) (layers F.Cu B.Cu) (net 6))
 (via (at 116.8631 125.5214) (size 0.8) (layers F.Cu B.Cu) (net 6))
 (segment (start 116.5362 125.5214) (end 116.8631 125.5214) (width 0.25) (layer B.Cu) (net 6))
 (segment (start 114.8276 127.23) (end 116.5362 125.5214) (width 0.25) (layer B.Cu) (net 6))
 (segment (start 114.234 127.23) (end 114.8276 127.23) (width 0.25) (layer B.Cu) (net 6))
 (segment (start 134.992919 123.19) (end 136.195 123.19) (width 0.25) (layer B.Cu) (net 6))
 (segment (start 132.854002 123.19) (end 134.992919 123.19) (width 0.25) (layer B.Cu) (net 6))
 (segment (start 131.662023 124.381979) (end 132.854002 123.19) (width 0.25) (layer B.Cu) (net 6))
 (segment (start 125.134821 124.381979) (end 131.662023 124.381979) (width 0.25) (layer B.Cu) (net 6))
 (segment (start 124.504 125.0128) (end 125.134821 124.381979) (width 0.25) (layer B.Cu) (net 6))
 (segment (start 114.1401 125.4239) (end 112.334 127.23) (width 0.25) (layer B.Cu) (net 5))
 (segment (start 117.1956 124.7961) (end 116.5627 124.7961) (width 0.25) (layer B.Cu) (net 5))
 (segment (start 112.334 127.23) (end 112.268 127.23) (width 0.25) (layer B.Cu) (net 5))
 (segment (start 115.935 125.4238) (end 115.935 125.4239) (width 0.25) (layer B.Cu) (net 5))
 (segment (start 116.5627 124.7961) (end 115.935 125.4238) (width 0.25) (layer B.Cu) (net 5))
 (segment (start 118.5827 122.9118) (end 118.5827 123.409) (width 0.25) (layer B.Cu) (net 5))
 (segment (start 118.5827 123.409) (end 117.1956 124.7961) (width 0.25) (layer B.Cu) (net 5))
 (segment (start 123.6747 122.2687) (end 119.2258 122.2687) (width 0.25) (layer B.Cu) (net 5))
 (segment (start 119.2258 122.2687) (end 118.5827 122.9118) (width 0.25) (layer B.Cu) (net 5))
 (segment (start 115.935 125.4239) (end 114.1401 125.4239) (width 0.25) (layer B.Cu) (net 5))
 (segment (start 124.723 123.317) (end 123.6747 122.2687) (width 0.25) (layer B.Cu) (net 5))
 (segment (start 130.556 123.19) (end 131.115 123.19) (width 0.25) (layer B.Cu) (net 5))
 (segment (start 129.33121 121.96521) (end 130.556 123.19) (width 0.25) (layer B.Cu) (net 5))
 (segment (start 126.07479 121.96521) (end 129.33121 121.96521) (width 0.25) (layer B.Cu) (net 5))
 (segment (start 124.723 123.317) (end 126.07479 121.96521) (width 0.25) (layer B.Cu) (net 5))
 (segment (start 115.842 128.524) (end 118.6055 125.7605) (width 0.25) (layer F.Cu) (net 4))
 (segment (start 118.6055 125.7605) (end 124.8292 125.7605) (width 0.25) (layer F.Cu) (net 4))
 (segment (start 124.8292 125.7605) (end 127.3997 123.19) (width 0.25) (layer F.Cu) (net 4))
 (segment (start 128.575 123.19) (end 127.3997 123.19) (width 0.25) (layer F.Cu) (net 4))
 (segment (start 124.469 127.889) (end 123.2761 129.0819) (width 0.25) (layer F.Cu) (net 13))
 (via (at 119.1849 129.0819) (size 0.8) (layers F.Cu B.Cu) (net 13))
 (segment (start 123.2761 129.0819) (end 119.1849 129.0819) (width 0.25) (layer F.Cu) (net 13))
 (segment (start 98.741 127.009) (end 99.441 127.009) (width 0.25) (layer B.Cu) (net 13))
 (segment (start 98.732 127) (end 98.741 127.009) (width 0.25) (layer B.Cu) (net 13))
 (segment (start 97.917 127) (end 98.732 127) (width 0.25) (layer B.Cu) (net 13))
 (segment (start 97.282 126.365) (end 97.917 127) (width 0.25) (layer B.Cu) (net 13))
 (segment (start 97.282 125.73) (end 97.282 126.365) (width 0.25) (layer B.Cu) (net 13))
 (segment (start 118.619215 129.0819) (end 118.257125 129.44399) (width 0.25) (layer B.Cu) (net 13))
 (segment (start 101.30099 129.44399) (end 99.441 127.584) (width 0.25) (layer B.Cu) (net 13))
 (segment (start 119.1849 129.0819) (end 118.619215 129.0819) (width 0.25) (layer B.Cu) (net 13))
 (segment (start 118.257125 129.44399) (end 101.30099 129.44399) (width 0.25) (layer B.Cu) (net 13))
 (segment (start 99.441 127.584) (end 99.441 127.009) (width 0.25) (layer B.Cu) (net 13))
 (segment (start 124.596 123.317) (end 123.1169 124.7961) (width 0.25) (layer F.Cu) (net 1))
 (segment (start 123.1169 124.7961) (end 116.5627 124.7961) (width 0.25) (layer F.Cu) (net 1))
 (segment (start 116.5627 124.7961) (end 115.5842 125.7746) (width 0.25) (layer F.Cu) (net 1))
 (segment (start 115.5842 125.7746) (end 106.5411 125.7746) (width 0.25) (layer F.Cu) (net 1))
 (segment (start 106.5411 125.7746) (end 105.7286 126.5871) (width 0.25) (layer F.Cu) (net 1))
 (segment (start 105.7286 126.5871) (end 105.7286 126.7097) (width 0.25) (layer F.Cu) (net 1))
 (segment (start 105.7286 126.7097) (end 104.2129 128.2254) (width 0.25) (layer F.Cu) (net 1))
 (segment (start 104.2129 128.2254) (end 94.6027 128.2254) (width 0.25) (layer F.Cu) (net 1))
 (segment (start 94.6027 128.2254) (end 92.1073 125.73) (width 0.25) (layer F.Cu) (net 1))
 (segment (start 90.932 125.73) (end 92.1073 125.73) (width 0.25) (layer F.Cu) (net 1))
 (segment (start 115.5566 122.9546) (end 116.332 123.73) (width 0.25) (layer B.Cu) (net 1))
 (segment (start 110.236 122.9546) (end 115.5566 122.9546) (width 0.25) (layer B.Cu) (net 1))
 (segment (start 110.236 123.73) (end 110.236 122.9546) (width 0.25) (layer B.Cu) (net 1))
 (segment (start 99.06 124.959) (end 99.06 123.952) (width 0.25) (layer B.Cu) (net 1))
 (segment (start 110.236 122.936) (end 110.236 123.73) (width 0.25) (layer B.Cu) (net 1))
 (segment (start 100.076 122.936) (end 110.236 122.936) (width 0.25) (layer B.Cu) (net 1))
 (segment (start 99.06 123.952) (end 100.076 122.936) (width 0.25) (layer B.Cu) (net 1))
 (segment (start 93.59 125.73) (end 90.932 125.73) (width 0.25) (layer B.Cu) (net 1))
 (segment (start 94.996 125.73) (end 93.59 125.73) (width 0.25) (layer B.Cu) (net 1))
 (segment (start 96.774 123.952) (end 94.996 125.73) (width 0.25) (layer B.Cu) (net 1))
 (segment (start 99.06 123.952) (end 96.774 123.952) (width 0.25) (layer B.Cu) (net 1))
 (segment (start 119.38 123.976) (end 119.38 125.2513) (width 0.25) (layer B.Cu) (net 12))
 (segment (start 119.38 125.2513) (end 118.3351 125.2513) (width 0.25) (layer B.Cu) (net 12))
 (segment (start 118.3351 125.2513) (end 116.332 127.2544) (width 0.25) (layer B.Cu) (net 12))
 (segment (start 116.332 127.2544) (end 116.332 127.73) (width 0.25) (layer B.Cu) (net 12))
 (segment (start 113.284 124.23) (end 112.5587 124.23) (width 0.25) (layer B.Cu) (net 11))
 (segment (start 112.5587 124.23) (end 110.236 126.5527) (width 0.25) (layer B.Cu) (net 11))
 (segment (start 110.236 126.5527) (end 110.236 127.73) (width 0.25) (layer B.Cu) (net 11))
 (segment (start 103.124 127) (end 104.3493 127) (width 0.25) (layer F.Cu) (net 14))
 (segment (start 113.91 122.809) (end 107.5447 122.809) (width 0.25) (layer F.Cu) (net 14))
 (segment (start 107.5447 122.809) (end 104.3493 126.0044) (width 0.25) (layer F.Cu) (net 14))
 (segment (start 104.3493 126.0044) (end 104.3493 127) (width 0.25) (layer F.Cu) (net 14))
 (segment (start 107.696 127) (end 108.9213 127) (width 0.25) (layer F.Cu) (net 15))
 (segment (start 113.792 128.524) (end 110.4453 128.524) (width 0.25) (layer F.Cu) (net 15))
 (segment (start 110.4453 128.524) (end 108.9213 127) (width 0.25) (layer F.Cu) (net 15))
 (segment (start 122.673 126.61) (end 125.603 126.61) (width 0.25) (layer B.Cu) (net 2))
 (segment (start 122.673 126.61) (end 122.673 123.317) (width 0.25) (layer B.Cu) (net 2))
 (segment (start 138.176 128.27) (end 135.636 125.73) (width 0.25) (layer B.Cu) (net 2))
 (segment (start 135.636 125.73) (end 133.655 125.73) (width 0.25) (layer B.Cu) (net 2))
 (segment (start 138.735 128.27) (end 138.176 128.27) (width 0.25) (layer B.Cu) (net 2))
 (segment (start 125.603 126.035) (end 126.797 124.841) (width 0.25) (layer B.Cu) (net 2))
 (segment (start 125.603 126.61) (end 125.603 126.035) (width 0.25) (layer B.Cu) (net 2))
 (segment (start 126.797 124.841) (end 129.159 124.841) (width 0.25) (layer B.Cu) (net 2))
 (segment (start 129.159 125.839) (end 129.159 124.841) (width 0.25) (layer B.Cu) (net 2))
 (segment (start 129.15 125.848) (end 129.159 125.839) (width 0.25) (layer B.Cu) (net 2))
 (segment (start 129.15 125.984) (end 129.15 125.848) (width 0.25) (layer B.Cu) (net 2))
 (segment (start 133.477 125.73) (end 133.655 125.73) (width 0.25) (layer B.Cu) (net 2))
 (segment (start 131.76318 124.83199) (end 131.77219 124.841) (width 0.25) (layer B.Cu) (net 2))
 (segment (start 132.588 124.841) (end 133.477 125.73) (width 0.25) (layer B.Cu) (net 2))
 (segment (start 131.77219 124.841) (end 132.588 124.841) (width 0.25) (layer B.Cu) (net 2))
 (segment (start 129.16801 124.83199) (end 131.76318 124.83199) (width 0.25) (layer B.Cu) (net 2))
 (segment (start 129.159 124.841) (end 129.16801 124.83199) (width 0.25) (layer B.Cu) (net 2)))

